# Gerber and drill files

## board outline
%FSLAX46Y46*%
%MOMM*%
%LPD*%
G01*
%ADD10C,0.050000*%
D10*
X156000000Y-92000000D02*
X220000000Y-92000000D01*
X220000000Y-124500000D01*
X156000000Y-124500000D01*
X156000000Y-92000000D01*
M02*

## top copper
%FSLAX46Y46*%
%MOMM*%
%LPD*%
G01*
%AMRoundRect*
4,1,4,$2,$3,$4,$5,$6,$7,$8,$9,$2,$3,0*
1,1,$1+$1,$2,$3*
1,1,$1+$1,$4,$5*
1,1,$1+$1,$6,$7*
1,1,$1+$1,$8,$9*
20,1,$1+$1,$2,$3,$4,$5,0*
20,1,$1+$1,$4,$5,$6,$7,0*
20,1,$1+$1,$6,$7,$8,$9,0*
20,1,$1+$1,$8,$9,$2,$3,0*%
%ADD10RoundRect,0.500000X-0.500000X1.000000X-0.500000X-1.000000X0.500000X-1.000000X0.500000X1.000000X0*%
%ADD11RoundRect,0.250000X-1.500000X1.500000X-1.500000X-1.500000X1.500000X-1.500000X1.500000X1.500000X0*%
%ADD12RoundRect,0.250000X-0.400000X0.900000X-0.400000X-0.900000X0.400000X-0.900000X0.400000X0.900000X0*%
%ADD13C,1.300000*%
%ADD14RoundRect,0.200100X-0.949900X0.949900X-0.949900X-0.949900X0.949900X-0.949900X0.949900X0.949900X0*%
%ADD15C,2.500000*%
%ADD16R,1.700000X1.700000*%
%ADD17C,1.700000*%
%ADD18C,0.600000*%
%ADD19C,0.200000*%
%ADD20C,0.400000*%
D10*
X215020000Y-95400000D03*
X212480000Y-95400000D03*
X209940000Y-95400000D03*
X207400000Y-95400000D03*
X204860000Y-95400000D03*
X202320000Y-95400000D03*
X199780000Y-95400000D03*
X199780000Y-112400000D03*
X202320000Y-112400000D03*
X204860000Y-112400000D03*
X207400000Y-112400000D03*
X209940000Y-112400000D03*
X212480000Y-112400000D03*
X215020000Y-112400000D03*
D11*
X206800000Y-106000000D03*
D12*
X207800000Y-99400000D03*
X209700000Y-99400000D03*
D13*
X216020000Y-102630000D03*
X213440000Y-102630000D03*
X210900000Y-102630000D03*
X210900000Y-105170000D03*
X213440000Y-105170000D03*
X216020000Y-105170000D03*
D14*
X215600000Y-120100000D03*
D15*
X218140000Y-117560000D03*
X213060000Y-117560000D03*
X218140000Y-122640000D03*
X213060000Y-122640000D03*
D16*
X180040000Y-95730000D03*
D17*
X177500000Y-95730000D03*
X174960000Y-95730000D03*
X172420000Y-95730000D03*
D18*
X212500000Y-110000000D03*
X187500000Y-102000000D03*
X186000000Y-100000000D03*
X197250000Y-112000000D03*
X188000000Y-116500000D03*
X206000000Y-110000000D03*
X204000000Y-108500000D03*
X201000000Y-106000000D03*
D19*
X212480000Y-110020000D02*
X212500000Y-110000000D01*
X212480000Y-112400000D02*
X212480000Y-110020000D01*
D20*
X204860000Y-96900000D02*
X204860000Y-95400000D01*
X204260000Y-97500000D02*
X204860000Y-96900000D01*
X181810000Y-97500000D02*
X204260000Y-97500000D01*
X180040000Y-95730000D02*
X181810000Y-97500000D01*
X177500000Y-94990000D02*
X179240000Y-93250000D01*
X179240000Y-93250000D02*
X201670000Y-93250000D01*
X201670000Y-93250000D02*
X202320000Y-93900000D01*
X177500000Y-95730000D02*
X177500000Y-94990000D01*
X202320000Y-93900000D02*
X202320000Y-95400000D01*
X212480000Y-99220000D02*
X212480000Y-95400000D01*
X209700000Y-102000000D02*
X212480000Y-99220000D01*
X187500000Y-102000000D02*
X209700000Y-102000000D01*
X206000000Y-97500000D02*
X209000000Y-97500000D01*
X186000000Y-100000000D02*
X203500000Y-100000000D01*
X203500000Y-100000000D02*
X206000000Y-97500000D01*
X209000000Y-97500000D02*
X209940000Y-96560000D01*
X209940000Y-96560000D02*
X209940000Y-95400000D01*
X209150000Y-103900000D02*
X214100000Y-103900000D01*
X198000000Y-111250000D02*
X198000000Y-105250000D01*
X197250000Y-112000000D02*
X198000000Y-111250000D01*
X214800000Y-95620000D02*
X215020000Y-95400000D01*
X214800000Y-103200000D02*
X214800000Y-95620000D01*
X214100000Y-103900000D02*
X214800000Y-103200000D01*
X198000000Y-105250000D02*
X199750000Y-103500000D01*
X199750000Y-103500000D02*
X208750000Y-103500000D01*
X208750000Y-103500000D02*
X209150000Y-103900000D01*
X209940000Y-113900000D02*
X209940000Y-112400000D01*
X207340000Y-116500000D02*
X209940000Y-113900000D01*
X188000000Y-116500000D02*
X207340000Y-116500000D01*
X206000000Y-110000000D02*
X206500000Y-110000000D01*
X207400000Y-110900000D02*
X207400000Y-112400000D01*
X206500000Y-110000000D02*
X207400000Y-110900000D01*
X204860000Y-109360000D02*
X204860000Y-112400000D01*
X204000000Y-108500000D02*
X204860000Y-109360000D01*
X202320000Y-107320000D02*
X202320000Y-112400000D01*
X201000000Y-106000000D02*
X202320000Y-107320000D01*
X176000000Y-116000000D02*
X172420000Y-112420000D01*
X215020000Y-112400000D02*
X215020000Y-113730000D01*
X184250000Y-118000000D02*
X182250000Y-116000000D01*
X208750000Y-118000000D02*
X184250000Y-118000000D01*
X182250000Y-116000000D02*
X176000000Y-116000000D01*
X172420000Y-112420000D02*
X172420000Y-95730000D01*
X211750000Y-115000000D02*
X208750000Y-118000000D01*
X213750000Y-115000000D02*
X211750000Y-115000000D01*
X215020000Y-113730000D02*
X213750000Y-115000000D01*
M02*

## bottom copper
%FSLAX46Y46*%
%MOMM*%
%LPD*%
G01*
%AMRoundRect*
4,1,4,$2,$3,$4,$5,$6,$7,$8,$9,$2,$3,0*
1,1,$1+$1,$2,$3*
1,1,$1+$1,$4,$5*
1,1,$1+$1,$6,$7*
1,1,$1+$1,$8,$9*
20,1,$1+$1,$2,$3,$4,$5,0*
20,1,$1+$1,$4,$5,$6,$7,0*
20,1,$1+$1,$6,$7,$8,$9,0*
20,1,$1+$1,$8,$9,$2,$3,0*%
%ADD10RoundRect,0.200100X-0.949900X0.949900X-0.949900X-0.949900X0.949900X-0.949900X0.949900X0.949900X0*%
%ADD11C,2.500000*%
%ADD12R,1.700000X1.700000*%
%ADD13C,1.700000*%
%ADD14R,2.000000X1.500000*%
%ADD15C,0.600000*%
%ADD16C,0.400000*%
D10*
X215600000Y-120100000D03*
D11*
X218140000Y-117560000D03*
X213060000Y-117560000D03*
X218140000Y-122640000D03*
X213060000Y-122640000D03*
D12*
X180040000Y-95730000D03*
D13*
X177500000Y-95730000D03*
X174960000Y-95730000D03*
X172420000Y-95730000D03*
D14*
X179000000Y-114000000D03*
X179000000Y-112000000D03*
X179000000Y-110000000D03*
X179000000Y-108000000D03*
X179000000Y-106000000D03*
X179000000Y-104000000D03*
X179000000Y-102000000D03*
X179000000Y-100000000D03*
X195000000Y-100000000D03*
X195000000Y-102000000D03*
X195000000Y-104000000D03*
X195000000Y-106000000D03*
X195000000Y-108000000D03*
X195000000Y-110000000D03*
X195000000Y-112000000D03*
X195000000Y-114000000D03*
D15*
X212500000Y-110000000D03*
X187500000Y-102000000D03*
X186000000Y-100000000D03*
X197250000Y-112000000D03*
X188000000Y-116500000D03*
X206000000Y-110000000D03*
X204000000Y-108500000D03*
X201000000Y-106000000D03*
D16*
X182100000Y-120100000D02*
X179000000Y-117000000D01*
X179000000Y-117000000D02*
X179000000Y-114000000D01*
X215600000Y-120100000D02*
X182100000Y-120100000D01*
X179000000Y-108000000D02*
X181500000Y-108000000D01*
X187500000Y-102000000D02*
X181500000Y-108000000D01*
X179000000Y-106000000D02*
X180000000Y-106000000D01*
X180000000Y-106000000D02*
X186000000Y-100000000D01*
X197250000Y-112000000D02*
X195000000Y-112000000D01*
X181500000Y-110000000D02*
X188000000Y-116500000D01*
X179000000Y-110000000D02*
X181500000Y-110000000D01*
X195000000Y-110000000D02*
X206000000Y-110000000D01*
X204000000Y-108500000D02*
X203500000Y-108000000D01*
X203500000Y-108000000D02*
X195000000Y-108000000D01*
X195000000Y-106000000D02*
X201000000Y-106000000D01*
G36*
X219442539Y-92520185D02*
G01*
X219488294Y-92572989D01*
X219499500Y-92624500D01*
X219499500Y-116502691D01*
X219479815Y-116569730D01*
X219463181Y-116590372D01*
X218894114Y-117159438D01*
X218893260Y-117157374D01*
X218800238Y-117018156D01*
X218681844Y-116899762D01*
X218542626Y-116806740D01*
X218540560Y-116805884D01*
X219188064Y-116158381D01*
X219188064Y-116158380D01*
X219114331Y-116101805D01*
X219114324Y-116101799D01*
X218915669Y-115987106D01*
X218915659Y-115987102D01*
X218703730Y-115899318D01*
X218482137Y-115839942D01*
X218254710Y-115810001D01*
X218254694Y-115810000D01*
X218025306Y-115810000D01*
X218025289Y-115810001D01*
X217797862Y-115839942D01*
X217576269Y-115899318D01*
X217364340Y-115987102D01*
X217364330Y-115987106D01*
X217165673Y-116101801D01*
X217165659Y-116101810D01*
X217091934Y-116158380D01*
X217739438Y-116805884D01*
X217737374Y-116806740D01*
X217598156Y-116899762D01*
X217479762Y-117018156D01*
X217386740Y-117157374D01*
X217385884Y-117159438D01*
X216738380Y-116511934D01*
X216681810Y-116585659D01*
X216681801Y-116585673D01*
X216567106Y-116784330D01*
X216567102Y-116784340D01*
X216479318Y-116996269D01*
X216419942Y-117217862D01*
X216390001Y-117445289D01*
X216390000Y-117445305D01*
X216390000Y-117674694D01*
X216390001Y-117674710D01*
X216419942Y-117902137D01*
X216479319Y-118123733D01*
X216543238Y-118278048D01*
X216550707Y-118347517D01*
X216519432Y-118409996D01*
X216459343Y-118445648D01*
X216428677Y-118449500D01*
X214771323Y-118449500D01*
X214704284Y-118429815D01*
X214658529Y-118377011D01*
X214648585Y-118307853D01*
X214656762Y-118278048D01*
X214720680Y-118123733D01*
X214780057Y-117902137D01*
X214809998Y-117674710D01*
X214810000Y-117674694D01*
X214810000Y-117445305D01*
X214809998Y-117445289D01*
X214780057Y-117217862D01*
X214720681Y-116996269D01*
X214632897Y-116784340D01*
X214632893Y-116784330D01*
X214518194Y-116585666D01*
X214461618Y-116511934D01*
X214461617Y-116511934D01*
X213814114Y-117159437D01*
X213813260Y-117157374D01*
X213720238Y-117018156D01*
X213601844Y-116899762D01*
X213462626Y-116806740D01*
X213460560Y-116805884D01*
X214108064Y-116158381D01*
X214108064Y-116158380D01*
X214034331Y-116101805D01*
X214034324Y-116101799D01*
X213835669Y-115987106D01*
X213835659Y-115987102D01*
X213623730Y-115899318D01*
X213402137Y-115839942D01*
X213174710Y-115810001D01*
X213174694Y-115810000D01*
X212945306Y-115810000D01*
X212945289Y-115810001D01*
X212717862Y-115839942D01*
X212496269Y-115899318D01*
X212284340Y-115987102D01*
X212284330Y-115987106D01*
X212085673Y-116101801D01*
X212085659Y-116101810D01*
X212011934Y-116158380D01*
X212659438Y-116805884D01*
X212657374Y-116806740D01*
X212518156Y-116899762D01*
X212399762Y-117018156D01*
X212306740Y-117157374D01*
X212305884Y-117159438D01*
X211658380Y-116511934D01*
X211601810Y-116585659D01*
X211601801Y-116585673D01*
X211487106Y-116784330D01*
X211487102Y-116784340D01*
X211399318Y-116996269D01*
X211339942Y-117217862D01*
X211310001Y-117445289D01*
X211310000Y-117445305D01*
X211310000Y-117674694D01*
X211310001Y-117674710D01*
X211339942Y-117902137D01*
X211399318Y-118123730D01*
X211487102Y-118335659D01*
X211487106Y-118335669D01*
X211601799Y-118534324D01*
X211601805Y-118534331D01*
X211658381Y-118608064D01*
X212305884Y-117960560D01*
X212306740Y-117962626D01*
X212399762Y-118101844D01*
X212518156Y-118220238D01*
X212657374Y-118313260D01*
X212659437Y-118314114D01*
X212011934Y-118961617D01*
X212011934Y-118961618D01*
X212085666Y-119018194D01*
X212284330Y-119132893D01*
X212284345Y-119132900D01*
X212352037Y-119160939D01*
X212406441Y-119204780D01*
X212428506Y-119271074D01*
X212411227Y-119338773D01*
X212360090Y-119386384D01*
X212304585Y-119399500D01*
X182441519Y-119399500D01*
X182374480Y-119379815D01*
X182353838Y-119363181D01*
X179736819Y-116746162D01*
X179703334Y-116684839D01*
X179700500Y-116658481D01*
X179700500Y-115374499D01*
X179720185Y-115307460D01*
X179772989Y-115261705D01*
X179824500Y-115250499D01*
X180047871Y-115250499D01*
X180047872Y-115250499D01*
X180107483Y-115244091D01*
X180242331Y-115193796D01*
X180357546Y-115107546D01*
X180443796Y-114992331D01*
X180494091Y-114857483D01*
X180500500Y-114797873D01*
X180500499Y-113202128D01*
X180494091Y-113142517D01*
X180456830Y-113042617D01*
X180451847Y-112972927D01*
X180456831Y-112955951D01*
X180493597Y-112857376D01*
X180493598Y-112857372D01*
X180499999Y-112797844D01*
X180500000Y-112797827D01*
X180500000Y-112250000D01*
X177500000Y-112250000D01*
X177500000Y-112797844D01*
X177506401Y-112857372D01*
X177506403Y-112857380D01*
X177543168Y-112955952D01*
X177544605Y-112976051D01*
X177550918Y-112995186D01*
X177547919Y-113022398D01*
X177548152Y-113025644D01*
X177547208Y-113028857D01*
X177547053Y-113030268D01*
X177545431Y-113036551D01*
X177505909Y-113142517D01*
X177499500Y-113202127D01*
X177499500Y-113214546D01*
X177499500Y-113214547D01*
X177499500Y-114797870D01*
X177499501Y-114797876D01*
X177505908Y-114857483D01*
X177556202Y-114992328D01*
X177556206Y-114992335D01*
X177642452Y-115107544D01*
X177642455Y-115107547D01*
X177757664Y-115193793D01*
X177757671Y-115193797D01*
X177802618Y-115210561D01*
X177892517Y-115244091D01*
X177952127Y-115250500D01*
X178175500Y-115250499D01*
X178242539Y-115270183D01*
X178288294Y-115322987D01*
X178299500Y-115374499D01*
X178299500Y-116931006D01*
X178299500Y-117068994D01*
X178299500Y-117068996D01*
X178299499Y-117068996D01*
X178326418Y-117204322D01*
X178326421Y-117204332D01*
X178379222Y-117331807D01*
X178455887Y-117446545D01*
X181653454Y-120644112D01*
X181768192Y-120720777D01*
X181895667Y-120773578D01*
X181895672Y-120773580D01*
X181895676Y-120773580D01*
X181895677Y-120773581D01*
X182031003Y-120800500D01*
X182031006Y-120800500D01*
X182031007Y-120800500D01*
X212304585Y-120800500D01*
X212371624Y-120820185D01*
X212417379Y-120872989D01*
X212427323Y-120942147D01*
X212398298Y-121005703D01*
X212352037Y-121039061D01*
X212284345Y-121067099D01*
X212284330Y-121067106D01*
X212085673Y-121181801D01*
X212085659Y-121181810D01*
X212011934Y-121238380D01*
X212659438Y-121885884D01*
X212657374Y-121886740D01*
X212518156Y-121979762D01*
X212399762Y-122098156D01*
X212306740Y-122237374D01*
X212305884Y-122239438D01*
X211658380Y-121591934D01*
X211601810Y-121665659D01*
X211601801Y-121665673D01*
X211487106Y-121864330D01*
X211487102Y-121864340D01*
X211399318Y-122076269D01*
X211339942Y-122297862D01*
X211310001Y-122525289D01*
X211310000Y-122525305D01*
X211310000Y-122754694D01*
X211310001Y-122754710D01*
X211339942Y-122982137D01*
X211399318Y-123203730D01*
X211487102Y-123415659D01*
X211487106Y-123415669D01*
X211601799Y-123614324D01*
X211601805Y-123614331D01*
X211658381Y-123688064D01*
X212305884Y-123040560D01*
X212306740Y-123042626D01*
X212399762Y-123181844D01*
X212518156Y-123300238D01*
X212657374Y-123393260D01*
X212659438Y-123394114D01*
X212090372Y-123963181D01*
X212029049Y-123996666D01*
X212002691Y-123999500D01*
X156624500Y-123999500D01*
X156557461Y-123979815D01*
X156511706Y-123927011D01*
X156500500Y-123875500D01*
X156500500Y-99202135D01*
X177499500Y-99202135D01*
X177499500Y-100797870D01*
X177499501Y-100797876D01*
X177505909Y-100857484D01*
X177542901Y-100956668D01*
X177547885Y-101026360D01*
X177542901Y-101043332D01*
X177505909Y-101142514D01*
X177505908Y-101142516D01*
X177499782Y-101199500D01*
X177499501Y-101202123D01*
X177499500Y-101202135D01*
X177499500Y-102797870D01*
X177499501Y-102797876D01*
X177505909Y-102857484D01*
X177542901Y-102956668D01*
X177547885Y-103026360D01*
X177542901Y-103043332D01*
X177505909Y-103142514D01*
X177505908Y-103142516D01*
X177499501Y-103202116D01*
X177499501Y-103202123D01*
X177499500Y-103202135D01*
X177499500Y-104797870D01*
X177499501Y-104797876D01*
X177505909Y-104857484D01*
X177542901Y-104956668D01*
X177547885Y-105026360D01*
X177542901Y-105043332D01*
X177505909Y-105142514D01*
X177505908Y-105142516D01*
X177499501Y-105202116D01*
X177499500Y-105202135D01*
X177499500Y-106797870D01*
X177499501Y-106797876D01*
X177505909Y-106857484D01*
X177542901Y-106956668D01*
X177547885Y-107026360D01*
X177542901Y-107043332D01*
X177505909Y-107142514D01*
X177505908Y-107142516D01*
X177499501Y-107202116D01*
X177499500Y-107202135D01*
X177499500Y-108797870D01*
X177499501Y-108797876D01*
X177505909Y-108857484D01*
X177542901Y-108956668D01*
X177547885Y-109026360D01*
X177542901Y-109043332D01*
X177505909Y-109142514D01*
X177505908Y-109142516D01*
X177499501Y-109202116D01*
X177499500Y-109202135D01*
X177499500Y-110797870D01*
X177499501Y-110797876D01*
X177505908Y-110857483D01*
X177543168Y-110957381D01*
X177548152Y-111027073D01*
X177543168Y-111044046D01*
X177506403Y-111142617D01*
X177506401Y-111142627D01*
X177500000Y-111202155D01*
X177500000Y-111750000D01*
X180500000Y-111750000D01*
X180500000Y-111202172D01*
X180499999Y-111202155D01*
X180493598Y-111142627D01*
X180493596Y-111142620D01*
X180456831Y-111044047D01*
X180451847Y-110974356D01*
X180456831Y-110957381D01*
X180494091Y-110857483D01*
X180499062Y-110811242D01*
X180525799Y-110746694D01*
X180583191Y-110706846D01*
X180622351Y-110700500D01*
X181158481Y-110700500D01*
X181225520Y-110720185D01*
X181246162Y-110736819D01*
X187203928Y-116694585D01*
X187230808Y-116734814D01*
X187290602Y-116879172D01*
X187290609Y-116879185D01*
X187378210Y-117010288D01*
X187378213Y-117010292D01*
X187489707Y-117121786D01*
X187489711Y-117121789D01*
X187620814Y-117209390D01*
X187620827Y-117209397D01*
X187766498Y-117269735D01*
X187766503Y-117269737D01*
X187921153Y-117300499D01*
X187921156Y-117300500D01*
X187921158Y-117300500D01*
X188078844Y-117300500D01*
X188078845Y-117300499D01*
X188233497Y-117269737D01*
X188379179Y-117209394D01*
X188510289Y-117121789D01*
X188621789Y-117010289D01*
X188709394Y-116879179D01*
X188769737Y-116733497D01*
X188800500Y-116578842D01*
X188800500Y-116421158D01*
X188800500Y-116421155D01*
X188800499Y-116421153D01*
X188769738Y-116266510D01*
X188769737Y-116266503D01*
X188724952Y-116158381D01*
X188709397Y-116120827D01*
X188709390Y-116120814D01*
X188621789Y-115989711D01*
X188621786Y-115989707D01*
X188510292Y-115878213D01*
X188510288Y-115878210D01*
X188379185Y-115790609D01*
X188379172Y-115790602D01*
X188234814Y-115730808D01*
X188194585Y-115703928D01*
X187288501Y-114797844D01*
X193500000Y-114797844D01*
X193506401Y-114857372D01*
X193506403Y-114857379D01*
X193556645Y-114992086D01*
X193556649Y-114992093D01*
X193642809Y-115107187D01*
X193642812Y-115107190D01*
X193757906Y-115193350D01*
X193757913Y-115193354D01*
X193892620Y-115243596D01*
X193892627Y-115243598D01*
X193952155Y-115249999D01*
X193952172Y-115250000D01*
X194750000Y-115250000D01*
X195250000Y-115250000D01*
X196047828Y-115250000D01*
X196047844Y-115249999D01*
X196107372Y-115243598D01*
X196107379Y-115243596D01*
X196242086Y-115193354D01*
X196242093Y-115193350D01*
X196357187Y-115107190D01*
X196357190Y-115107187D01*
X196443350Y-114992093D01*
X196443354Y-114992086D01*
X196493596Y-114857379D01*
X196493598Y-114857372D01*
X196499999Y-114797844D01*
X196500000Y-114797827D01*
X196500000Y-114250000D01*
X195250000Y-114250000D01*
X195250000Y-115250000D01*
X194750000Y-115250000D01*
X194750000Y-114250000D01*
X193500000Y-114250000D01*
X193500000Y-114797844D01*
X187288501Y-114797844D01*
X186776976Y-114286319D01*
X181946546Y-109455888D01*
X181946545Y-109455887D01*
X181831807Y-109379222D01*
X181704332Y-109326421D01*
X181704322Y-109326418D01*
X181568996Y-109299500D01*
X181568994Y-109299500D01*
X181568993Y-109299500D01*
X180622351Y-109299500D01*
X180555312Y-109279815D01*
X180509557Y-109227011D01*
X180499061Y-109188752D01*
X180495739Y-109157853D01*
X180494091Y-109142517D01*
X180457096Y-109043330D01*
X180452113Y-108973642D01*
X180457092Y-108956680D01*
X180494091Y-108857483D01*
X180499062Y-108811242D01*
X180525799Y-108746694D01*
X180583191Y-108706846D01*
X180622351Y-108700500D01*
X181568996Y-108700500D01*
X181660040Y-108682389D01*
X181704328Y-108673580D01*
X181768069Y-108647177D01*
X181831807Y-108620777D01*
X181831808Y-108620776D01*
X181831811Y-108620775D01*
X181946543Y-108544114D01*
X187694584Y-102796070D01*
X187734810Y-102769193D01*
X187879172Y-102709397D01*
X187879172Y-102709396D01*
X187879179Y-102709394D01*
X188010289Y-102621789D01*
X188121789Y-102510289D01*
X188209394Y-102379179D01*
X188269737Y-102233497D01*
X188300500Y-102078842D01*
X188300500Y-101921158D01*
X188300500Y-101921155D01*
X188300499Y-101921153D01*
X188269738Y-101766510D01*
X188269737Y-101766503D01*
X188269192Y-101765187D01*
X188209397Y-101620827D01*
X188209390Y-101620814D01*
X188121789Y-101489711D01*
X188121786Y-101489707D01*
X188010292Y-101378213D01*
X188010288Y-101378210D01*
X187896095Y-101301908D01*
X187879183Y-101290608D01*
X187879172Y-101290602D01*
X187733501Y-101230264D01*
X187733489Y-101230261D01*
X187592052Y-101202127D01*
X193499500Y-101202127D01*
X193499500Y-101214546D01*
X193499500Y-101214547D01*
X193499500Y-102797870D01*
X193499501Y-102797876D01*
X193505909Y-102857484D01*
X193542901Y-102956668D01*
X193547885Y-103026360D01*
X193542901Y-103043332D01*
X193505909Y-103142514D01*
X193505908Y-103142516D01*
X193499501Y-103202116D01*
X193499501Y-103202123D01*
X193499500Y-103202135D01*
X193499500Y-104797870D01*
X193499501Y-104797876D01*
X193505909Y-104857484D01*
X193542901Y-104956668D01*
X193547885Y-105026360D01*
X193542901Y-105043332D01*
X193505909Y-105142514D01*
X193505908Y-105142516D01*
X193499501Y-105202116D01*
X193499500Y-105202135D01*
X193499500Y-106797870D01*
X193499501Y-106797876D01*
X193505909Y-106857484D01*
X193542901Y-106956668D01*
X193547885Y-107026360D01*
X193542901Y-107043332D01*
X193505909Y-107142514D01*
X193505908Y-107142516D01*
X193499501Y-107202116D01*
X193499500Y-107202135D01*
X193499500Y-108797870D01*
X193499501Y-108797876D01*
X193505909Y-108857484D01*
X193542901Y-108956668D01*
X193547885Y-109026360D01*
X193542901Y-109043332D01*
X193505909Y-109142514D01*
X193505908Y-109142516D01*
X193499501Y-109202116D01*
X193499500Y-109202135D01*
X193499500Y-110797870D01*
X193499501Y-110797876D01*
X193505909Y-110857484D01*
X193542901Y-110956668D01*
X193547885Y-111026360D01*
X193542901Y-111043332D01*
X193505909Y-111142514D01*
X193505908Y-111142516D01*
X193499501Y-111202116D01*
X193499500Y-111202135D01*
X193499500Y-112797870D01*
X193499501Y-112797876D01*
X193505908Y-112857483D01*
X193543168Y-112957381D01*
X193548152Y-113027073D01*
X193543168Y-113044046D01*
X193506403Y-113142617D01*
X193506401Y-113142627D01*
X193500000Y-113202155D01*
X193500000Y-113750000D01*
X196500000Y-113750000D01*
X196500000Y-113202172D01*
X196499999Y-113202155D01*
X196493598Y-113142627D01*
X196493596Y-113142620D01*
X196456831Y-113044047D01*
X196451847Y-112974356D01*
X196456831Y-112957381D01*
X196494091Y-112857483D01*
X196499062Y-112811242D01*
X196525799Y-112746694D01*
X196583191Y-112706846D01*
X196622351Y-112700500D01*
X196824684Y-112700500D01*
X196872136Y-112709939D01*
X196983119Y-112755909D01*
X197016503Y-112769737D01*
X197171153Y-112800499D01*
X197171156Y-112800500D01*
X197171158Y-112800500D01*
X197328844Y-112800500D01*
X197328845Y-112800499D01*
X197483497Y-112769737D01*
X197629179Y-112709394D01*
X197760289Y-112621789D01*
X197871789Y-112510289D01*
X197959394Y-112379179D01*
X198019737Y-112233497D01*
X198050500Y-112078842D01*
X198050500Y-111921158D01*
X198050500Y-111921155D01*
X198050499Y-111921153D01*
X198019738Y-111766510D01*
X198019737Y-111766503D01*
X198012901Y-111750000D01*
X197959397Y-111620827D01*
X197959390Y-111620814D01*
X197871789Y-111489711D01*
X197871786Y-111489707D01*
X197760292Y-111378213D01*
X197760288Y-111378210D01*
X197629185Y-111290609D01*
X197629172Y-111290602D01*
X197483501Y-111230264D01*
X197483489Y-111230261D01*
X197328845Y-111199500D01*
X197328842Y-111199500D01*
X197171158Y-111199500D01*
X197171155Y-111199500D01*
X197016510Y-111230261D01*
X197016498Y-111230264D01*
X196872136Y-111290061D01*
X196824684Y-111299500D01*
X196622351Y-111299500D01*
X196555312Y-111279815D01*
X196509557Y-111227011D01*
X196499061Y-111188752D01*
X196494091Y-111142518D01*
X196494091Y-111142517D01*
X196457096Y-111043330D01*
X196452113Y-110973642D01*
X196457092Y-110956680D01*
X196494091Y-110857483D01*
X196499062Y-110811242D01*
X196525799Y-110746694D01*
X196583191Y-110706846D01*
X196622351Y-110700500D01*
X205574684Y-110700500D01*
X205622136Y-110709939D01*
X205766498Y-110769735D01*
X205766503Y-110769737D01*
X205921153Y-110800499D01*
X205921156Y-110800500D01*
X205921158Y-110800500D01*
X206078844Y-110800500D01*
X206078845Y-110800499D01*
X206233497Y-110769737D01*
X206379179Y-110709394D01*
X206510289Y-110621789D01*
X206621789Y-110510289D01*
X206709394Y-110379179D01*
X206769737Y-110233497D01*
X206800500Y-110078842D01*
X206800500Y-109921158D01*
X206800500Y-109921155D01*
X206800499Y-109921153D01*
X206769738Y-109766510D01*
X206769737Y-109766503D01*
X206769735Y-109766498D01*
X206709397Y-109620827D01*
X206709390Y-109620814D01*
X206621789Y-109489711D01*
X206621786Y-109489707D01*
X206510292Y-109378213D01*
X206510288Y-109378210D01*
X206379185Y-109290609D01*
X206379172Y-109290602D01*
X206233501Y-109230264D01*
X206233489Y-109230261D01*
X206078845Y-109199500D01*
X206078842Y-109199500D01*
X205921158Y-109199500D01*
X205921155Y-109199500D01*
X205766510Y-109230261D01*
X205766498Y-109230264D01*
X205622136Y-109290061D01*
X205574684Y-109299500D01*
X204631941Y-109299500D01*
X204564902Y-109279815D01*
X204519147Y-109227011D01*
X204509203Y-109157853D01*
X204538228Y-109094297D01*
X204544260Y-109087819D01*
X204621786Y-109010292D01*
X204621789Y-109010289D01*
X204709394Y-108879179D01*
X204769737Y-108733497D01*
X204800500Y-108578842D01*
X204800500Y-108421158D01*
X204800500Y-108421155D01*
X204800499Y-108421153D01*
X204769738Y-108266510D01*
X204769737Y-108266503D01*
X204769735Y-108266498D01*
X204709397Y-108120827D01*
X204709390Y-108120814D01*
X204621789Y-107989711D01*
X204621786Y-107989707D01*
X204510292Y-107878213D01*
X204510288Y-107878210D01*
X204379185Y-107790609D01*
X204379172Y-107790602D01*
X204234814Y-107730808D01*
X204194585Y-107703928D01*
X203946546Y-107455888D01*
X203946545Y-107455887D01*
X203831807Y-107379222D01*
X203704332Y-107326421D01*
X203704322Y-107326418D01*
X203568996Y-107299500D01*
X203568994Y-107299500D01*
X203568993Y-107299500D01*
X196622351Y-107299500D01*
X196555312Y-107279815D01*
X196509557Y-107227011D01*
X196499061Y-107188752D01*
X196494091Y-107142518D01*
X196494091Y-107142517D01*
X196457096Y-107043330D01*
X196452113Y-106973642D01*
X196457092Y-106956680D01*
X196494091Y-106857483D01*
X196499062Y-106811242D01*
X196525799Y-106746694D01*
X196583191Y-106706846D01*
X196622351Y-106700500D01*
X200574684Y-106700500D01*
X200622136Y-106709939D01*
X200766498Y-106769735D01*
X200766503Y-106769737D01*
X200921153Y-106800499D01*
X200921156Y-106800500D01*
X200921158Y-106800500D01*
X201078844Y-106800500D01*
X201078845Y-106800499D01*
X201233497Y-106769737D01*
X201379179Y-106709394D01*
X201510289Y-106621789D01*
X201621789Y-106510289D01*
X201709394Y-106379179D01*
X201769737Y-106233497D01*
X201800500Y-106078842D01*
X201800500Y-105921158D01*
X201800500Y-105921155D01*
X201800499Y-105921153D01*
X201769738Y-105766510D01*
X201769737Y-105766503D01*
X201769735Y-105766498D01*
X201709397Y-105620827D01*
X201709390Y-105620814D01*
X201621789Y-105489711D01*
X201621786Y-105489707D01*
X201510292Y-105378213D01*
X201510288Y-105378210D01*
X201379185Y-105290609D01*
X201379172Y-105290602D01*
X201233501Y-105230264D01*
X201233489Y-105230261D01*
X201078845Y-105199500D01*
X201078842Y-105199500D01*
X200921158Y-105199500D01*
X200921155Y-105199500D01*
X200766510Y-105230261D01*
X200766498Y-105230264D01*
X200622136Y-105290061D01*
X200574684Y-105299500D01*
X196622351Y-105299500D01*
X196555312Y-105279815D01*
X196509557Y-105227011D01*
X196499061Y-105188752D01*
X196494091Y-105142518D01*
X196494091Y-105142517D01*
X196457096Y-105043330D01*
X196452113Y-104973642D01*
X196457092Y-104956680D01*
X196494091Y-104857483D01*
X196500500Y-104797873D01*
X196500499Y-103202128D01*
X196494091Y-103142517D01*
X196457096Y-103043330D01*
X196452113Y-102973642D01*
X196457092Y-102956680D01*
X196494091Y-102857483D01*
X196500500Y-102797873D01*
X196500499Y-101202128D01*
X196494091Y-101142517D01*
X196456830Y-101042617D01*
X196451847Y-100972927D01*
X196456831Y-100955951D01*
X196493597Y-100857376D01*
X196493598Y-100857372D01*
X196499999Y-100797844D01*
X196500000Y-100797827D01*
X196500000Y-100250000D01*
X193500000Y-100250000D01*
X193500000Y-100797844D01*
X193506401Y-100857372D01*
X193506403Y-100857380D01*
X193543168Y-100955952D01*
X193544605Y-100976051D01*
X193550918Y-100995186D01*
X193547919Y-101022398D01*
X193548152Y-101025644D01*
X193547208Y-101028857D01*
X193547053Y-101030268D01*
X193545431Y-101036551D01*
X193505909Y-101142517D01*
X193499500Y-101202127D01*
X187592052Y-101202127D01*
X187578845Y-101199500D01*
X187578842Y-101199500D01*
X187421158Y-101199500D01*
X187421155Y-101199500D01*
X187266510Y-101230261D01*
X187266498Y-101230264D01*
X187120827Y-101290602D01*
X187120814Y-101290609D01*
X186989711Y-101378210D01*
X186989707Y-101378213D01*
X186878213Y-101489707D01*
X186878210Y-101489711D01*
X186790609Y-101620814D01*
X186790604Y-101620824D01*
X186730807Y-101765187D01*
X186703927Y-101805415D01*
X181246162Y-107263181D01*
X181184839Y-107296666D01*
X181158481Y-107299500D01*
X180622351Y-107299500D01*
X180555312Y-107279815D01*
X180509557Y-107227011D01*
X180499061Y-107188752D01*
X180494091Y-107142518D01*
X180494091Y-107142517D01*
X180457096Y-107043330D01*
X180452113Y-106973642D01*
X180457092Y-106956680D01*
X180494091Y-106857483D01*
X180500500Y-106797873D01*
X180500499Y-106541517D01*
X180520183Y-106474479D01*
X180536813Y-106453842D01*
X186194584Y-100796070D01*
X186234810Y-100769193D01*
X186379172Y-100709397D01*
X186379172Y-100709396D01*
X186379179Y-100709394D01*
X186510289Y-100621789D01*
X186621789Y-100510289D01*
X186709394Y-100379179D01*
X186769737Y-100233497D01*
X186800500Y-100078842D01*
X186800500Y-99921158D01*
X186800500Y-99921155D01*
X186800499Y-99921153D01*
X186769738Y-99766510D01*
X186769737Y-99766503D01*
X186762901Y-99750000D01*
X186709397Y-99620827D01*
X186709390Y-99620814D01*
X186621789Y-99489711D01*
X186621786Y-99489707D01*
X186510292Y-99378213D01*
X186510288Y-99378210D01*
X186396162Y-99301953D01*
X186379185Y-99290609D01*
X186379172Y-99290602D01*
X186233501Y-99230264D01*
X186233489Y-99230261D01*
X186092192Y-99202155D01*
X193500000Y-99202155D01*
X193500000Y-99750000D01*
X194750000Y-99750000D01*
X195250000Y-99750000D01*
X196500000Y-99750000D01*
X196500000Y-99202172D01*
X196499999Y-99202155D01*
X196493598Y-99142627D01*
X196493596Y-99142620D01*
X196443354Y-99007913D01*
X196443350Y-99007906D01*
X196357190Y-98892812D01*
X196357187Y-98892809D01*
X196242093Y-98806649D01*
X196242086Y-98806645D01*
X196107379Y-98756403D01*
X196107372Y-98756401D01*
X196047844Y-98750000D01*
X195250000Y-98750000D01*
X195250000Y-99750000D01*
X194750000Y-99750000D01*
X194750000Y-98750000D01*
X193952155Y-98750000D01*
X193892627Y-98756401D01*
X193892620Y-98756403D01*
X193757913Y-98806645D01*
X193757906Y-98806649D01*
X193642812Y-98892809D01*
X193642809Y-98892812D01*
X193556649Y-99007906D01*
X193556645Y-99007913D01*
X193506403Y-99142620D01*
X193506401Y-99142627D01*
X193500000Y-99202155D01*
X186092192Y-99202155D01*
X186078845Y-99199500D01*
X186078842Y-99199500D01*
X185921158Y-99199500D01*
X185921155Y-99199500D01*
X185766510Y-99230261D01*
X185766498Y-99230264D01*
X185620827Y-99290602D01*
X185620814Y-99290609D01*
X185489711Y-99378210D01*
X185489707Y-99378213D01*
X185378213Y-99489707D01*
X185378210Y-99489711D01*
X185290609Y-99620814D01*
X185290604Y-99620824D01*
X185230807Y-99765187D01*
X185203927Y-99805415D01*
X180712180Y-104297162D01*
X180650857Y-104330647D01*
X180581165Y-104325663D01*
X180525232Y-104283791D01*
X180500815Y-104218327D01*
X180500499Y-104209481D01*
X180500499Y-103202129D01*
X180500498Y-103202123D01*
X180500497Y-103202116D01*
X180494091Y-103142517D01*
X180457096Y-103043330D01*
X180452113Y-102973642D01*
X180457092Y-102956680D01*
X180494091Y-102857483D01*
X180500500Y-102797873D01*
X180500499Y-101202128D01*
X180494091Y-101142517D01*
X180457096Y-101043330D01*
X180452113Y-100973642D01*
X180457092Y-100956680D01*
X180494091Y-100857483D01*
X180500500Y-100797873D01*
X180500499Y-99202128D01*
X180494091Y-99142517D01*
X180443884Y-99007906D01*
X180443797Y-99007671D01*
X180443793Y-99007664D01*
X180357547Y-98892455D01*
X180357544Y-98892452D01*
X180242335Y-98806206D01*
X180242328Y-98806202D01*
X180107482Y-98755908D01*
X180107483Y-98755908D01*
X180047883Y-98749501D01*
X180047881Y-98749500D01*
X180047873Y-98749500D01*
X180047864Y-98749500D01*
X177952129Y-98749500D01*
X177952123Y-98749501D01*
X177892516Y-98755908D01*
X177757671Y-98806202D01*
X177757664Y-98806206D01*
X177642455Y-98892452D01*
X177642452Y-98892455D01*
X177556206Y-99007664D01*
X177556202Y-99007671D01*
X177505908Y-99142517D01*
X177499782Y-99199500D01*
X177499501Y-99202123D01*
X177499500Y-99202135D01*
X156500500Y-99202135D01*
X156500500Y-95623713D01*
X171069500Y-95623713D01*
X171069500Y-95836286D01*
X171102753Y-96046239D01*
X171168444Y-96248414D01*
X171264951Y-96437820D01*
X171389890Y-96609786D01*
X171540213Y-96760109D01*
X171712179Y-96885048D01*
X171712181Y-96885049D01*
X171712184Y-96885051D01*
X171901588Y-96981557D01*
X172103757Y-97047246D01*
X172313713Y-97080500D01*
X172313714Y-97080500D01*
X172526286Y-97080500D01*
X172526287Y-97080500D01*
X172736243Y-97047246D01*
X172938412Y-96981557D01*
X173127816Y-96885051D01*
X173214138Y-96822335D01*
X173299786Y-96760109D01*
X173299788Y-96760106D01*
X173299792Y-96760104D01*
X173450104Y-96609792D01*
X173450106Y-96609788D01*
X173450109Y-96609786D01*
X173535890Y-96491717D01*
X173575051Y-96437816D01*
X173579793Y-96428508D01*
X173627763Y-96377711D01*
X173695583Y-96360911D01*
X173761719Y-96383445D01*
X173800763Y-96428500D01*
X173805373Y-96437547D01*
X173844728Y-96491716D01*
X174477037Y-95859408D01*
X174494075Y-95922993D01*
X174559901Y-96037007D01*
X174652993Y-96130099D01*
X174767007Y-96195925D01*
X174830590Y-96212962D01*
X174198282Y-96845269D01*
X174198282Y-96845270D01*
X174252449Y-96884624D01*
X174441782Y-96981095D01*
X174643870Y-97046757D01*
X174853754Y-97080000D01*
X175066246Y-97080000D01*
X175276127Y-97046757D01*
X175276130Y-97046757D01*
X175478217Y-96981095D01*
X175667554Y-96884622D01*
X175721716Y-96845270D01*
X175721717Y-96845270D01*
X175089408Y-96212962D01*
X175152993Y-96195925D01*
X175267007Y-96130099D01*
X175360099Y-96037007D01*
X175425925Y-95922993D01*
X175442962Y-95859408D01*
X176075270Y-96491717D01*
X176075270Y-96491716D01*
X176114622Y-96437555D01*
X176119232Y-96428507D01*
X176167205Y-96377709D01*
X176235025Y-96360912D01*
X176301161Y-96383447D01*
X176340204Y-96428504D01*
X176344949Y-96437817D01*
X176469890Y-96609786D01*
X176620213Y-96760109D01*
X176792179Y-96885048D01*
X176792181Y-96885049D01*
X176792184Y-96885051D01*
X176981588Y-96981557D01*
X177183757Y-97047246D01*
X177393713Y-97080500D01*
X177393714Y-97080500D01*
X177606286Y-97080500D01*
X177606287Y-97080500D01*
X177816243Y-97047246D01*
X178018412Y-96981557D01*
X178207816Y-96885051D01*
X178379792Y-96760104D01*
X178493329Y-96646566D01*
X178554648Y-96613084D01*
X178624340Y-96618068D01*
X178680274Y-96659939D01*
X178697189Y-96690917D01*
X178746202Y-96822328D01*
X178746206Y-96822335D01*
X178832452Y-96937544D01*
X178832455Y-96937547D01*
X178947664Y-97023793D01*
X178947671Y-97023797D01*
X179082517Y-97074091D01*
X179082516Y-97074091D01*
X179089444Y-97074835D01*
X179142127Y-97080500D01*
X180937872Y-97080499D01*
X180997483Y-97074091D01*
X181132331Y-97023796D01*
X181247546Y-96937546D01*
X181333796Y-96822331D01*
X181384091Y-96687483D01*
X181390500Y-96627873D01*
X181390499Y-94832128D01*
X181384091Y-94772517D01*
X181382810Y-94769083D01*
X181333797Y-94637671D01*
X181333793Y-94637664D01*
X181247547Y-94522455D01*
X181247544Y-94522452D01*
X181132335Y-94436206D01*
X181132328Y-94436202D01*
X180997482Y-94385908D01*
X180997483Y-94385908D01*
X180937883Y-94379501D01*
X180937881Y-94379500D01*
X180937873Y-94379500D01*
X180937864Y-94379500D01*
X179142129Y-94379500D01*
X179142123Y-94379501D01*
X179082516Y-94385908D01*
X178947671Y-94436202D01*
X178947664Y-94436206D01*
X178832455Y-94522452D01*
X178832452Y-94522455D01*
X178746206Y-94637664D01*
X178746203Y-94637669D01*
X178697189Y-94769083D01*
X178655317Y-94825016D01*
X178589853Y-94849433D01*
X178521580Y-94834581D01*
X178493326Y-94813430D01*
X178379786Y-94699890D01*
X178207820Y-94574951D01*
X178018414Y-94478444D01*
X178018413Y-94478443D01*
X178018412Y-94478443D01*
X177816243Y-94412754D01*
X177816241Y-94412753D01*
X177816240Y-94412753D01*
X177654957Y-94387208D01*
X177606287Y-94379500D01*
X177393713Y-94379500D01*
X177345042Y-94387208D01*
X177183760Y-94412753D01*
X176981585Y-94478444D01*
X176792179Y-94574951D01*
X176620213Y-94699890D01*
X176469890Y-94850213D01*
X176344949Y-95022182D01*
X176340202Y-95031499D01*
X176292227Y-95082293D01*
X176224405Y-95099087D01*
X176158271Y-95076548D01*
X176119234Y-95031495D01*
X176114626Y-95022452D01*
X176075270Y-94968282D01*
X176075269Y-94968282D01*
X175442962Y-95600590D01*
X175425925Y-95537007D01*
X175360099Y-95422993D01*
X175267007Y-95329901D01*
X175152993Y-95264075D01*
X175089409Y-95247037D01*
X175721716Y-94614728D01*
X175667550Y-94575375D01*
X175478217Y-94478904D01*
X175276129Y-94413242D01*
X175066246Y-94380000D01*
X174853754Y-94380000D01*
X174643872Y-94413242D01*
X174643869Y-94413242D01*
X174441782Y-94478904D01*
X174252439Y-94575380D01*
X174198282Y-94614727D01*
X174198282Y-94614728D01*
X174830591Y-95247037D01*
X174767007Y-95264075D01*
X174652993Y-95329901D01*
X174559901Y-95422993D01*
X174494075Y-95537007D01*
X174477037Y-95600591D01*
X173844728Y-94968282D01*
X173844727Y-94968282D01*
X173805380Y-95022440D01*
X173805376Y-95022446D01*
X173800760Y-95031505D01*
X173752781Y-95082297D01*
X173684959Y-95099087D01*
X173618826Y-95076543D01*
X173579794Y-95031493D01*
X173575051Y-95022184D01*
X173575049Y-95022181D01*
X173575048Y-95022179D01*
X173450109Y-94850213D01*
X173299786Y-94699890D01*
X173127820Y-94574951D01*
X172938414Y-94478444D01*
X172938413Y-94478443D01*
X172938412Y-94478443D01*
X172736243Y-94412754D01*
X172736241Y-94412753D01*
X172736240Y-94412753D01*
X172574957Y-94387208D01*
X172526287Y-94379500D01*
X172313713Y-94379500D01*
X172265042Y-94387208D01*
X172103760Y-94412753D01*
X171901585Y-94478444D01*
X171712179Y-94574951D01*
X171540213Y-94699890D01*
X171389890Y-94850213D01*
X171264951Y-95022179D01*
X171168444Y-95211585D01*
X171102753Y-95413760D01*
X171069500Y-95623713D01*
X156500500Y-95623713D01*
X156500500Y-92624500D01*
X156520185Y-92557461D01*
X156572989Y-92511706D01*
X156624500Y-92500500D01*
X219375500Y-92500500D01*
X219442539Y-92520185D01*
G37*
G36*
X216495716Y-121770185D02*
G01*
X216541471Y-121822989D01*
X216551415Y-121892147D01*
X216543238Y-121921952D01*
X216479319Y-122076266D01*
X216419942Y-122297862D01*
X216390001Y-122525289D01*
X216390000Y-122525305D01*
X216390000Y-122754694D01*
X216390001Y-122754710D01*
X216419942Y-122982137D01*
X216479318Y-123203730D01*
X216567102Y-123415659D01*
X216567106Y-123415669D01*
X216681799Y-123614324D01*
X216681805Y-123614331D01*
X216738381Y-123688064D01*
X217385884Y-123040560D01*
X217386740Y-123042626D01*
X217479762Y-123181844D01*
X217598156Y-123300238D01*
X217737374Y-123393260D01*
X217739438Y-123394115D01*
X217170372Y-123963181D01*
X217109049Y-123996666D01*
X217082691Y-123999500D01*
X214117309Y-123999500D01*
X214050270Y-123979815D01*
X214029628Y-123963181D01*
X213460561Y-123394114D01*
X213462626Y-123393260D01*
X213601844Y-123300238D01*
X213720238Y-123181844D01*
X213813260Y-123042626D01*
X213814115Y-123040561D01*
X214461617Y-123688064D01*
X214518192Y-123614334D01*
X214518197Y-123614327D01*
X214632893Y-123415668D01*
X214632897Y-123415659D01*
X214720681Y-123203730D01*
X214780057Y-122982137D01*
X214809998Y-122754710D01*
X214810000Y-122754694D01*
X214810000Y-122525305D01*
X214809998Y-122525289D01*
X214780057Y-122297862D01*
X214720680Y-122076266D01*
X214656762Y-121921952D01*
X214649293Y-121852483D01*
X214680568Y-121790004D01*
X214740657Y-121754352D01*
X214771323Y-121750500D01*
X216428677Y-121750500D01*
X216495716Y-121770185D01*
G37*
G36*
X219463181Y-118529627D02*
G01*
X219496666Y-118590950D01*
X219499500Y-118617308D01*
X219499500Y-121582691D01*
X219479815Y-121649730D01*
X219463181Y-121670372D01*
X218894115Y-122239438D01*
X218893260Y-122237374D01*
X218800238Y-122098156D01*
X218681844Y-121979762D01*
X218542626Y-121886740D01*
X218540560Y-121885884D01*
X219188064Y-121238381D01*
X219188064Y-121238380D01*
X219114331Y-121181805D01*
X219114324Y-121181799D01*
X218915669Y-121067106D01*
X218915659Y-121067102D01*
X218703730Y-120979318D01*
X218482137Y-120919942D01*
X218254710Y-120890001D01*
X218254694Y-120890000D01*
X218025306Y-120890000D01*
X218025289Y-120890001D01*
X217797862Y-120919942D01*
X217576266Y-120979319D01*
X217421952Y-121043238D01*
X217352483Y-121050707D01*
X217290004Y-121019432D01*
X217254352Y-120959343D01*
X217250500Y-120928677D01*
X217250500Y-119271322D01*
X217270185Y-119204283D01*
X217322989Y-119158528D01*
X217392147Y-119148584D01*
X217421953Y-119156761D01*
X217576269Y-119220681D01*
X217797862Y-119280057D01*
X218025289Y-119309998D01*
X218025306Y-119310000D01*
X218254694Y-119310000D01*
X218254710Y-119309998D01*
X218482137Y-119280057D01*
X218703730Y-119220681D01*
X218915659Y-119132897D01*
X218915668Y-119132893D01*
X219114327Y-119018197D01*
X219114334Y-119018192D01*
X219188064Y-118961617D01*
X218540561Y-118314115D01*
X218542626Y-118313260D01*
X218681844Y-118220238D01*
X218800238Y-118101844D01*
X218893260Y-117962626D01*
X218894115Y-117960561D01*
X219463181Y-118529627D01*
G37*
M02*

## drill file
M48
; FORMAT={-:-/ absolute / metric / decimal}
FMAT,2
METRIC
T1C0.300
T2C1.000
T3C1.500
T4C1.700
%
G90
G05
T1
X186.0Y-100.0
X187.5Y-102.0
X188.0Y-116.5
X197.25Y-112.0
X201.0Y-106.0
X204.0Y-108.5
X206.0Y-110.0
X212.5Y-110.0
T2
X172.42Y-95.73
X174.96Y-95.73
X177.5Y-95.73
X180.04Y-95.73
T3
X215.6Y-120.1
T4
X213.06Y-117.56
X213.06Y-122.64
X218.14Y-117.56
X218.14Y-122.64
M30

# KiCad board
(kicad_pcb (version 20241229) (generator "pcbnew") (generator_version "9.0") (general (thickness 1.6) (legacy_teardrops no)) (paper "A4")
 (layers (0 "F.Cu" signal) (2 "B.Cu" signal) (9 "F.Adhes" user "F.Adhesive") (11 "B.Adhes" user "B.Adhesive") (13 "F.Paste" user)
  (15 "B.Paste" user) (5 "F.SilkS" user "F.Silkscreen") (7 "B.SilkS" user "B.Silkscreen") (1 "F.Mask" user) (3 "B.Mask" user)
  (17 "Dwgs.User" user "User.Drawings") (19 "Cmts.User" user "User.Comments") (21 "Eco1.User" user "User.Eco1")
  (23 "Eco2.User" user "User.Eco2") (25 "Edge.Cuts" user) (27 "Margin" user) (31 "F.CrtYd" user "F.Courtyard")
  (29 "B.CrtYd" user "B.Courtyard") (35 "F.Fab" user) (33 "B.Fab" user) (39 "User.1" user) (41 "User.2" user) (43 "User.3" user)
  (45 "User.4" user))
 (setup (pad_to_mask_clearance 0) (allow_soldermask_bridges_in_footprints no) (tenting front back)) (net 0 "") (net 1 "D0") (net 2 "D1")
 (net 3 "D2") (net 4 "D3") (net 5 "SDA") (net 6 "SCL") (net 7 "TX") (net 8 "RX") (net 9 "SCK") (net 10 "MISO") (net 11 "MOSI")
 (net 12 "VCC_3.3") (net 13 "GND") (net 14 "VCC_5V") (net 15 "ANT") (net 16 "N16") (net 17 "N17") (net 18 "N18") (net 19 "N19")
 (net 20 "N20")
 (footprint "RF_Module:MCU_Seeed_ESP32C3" (layer "F.Cu") (at 207.4 103.9 -90)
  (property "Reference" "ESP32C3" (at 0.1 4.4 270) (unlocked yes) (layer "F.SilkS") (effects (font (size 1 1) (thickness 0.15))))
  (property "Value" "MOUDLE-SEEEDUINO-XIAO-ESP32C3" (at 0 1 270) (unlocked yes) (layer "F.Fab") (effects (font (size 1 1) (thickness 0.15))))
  (pad "" smd roundrect (at 1.1 -0.4 270) (size 1.5 1.5) (layers "F.Paste") (roundrect_rratio 0.1666666667))
  (pad "" smd roundrect (at 1.1 1.6 270) (size 1.5 1.5) (layers "F.Paste") (roundrect_rratio 0.1666666667))
  (pad "" smd roundrect (at 3.1 -0.4 270) (size 1.5 1.5) (layers "F.Paste") (roundrect_rratio 0.1666666667))
  (pad "" smd roundrect (at 3.1 1.6 270) (size 1.5 1.5) (layers "F.Paste") (roundrect_rratio 0.1666666667))
  (pad "1" smd roundrect (at -8.5 -7.62 270) (size 3 2) (layers "F.Cu" "F.Mask" "F.Paste") (roundrect_rratio 0.25) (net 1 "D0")
   (thermal_bridge_angle 45))
  (pad "2" smd roundrect (at -8.5 -5.08 270) (size 3 2) (layers "F.Cu" "F.Mask" "F.Paste") (roundrect_rratio 0.25) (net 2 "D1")
   (thermal_bridge_angle 45))
  (pad "3" smd roundrect (at -8.5 -2.54 270) (size 3 2) (layers "F.Cu" "F.Mask" "F.Paste") (roundrect_rratio 0.25) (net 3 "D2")
   (thermal_bridge_angle 45))
  (pad "4" smd roundrect (at -8.5 0 270) (size 3 2) (layers "F.Cu" "F.Mask" "F.Paste") (roundrect_rratio 0.25) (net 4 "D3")
   (thermal_bridge_angle 45))
  (pad "5" smd roundrect (at -8.5 2.54 270) (size 3 2) (layers "F.Cu" "F.Mask" "F.Paste") (roundrect_rratio 0.25) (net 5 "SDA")
   (thermal_bridge_angle 45))
  (pad "6" smd roundrect (at -8.5 5.08 270) (size 3 2) (layers "F.Cu" "F.Mask" "F.Paste") (roundrect_rratio 0.25) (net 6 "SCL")
   (thermal_bridge_angle 45))
  (pad "7" smd roundrect (at -8.5 7.62 270) (size 3 2) (layers "F.Cu" "F.Mask" "F.Paste") (roundrect_rratio 0.25) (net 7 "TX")
   (thermal_bridge_angle 45))
  (pad "8" smd roundrect (at 8.5 7.62 270) (size 3 2) (layers "F.Cu" "F.Mask" "F.Paste") (roundrect_rratio 0.25) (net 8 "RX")
   (thermal_bridge_angle 45))
  (pad "9" smd roundrect (at 8.5 5.08 270) (size 3 2) (layers "F.Cu" "F.Mask" "F.Paste") (roundrect_rratio 0.25) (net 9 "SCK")
   (thermal_bridge_angle 45))
  (pad "10" smd roundrect (at 8.5 2.54 270) (size 3 2) (layers "F.Cu" "F.Mask" "F.Paste") (roundrect_rratio 0.25) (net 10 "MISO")
   (thermal_bridge_angle 45))
  (pad "11" smd roundrect (at 8.5 0 270) (size 3 2) (layers "F.Cu" "F.Mask" "F.Paste") (roundrect_rratio 0.25) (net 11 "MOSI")
   (thermal_bridge_angle 45))
  (pad "12" smd roundrect (at 8.5 -2.54 270) (size 3 2) (layers "F.Cu" "F.Mask" "F.Paste") (roundrect_rratio 0.25) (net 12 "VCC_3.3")
   (thermal_bridge_angle 45))
  (pad "13" smd roundrect (at 8.5 -5.08 270) (size 3 2) (layers "F.Cu" "F.Mask" "F.Paste") (roundrect_rratio 0.25) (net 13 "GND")
   (thermal_bridge_angle 45))
  (pad "14" smd roundrect (at 8.5 -7.62 270) (size 3 2) (layers "F.Cu" "F.Mask" "F.Paste") (roundrect_rratio 0.25) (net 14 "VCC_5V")
   (thermal_bridge_angle 45))
  (pad "15" smd roundrect (at 2.1 0.6 270) (size 3.5 3.5) (layers "F.Cu" "F.Mask") (roundrect_rratio 0.07142857143))
  (pad "16" smd roundrect (at -4.5 -0.4 270) (size 2.3 1.3) (layers "F.Cu" "F.Mask" "F.Paste") (roundrect_rratio 0.1923076923))
  (pad "17" smd roundrect (at -4.5 -2.3 270) (size 2.3 1.3) (layers "F.Cu" "F.Mask" "F.Paste") (roundrect_rratio 0.1923076923))
  (pad "18" smd circle (at -1.27 -8.62 270) (size 1.3 1.3) (layers "F.Cu" "F.Mask" "F.Paste"))
  (pad "19" smd circle (at -1.27 -6.04 270) (size 1.3 1.3) (layers "F.Cu" "F.Mask" "F.Paste"))
  (pad "20" smd circle (at -1.27 -3.5 270) (size 1.3 1.3) (layers "F.Cu" "F.Mask" "F.Paste"))
  (pad "21" smd circle (at 1.27 -3.5 270) (size 1.3 1.3) (layers "F.Cu" "F.Mask" "F.Paste"))
  (pad "22" smd circle (at 1.27 -6.04 270) (size 1.3 1.3) (layers "F.Cu" "F.Mask" "F.Paste"))
  (pad "23" smd circle (at 1.27 -8.62 270) (size 1.3 1.3) (layers "F.Cu" "F.Mask" "F.Paste")))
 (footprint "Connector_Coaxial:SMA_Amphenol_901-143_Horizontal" (layer "F.Cu") (at 215.6 120.1 -90)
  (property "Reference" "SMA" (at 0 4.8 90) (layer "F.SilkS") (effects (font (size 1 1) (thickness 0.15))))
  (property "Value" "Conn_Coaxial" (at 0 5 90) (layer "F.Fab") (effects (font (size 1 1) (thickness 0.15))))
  (pad "1" thru_hole roundrect (at 0 0 270) (size 2.3 2.3) (drill 1.5) (layers "*.Cu" "*.Mask") (remove_unused_layers yes)
   (keep_end_layers yes) (zone_layer_connections) (roundrect_rratio 0.087) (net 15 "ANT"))
  (pad "2" thru_hole circle (at -2.54 -2.54 270) (size 2.5 2.5) (drill 1.7) (layers "*.Cu" "*.Mask") (remove_unused_layers yes)
   (keep_end_layers yes) (zone_layer_connections) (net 13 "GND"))
  (pad "2" thru_hole circle (at -2.54 2.54 270) (size 2.5 2.5) (drill 1.7) (layers "*.Cu" "*.Mask") (remove_unused_layers yes)
   (keep_end_layers yes) (zone_layer_connections) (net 13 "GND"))
  (pad "2" thru_hole circle (at 2.54 -2.54 270) (size 2.5 2.5) (drill 1.7) (layers "*.Cu" "*.Mask") (remove_unused_layers yes)
   (keep_end_layers yes) (zone_layer_connections) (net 13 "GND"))
  (pad "2" thru_hole circle (at 2.54 2.54 270) (size 2.5 2.5) (drill 1.7) (layers "*.Cu" "*.Mask") (remove_unused_layers yes)
   (keep_end_layers yes) (zone_layer_connections) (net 13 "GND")))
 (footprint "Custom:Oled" (layer "F.Cu") (at 176 102)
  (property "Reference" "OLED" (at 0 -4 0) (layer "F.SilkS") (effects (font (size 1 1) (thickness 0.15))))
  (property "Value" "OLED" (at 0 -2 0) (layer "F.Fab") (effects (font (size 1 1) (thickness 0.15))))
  (pad "1" thru_hole rect (at 4.04 -6.27 270) (size 1.7 1.7) (drill 1) (layers "*.Cu" "*.Mask") (remove_unused_layers no) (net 5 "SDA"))
  (pad "2" thru_hole circle (at 1.5 -6.27 270) (size 1.7 1.7) (drill 1) (layers "*.Cu" "*.Mask") (remove_unused_layers no) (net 6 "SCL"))
  (pad "3" thru_hole circle (at -1.04 -6.27 270) (size 1.7 1.7) (drill 1) (layers "*.Cu" "*.Mask") (remove_unused_layers no) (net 13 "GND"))
  (pad "4" thru_hole circle (at -3.58 -6.27 270) (size 1.7 1.7) (drill 1) (layers "*.Cu" "*.Mask") (remove_unused_layers no)
   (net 14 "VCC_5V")))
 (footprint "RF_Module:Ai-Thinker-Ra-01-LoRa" (layer "B.Cu") (at 187 107)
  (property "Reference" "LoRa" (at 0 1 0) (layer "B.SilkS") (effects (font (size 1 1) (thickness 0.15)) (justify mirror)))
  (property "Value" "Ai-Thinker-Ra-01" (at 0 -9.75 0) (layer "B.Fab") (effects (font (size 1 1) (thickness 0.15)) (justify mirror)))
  (pad "1" smd rect (at -8 7) (size 2 1.5) (layers "B.Cu" "B.Mask" "B.Paste") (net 15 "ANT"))
  (pad "2" smd rect (at -8 5) (size 2 1.5) (layers "B.Cu" "B.Mask" "B.Paste") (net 13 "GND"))
  (pad "3" smd rect (at -8 3) (size 2 1.5) (layers "B.Cu" "B.Mask" "B.Paste") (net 12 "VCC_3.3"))
  (pad "4" smd rect (at -8 1) (size 2 1.5) (layers "B.Cu" "B.Mask" "B.Paste") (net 2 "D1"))
  (pad "5" smd rect (at -8 -1) (size 2 1.5) (layers "B.Cu" "B.Mask" "B.Paste") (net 3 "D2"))
  (pad "6" smd rect (at -8 -3) (size 2 1.5) (layers "B.Cu" "B.Mask" "B.Paste") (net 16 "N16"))
  (pad "7" smd rect (at -8 -5) (size 2 1.5) (layers "B.Cu" "B.Mask" "B.Paste") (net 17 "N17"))
  (pad "8" smd rect (at -8 -7) (size 2 1.5) (layers "B.Cu" "B.Mask" "B.Paste") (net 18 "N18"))
  (pad "9" smd rect (at 8 -7) (size 2 1.5) (layers "B.Cu" "B.Mask" "B.Paste") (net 13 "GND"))
  (pad "10" smd rect (at 8 -5) (size 2 1.5) (layers "B.Cu" "B.Mask" "B.Paste") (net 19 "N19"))
  (pad "11" smd rect (at 8 -3) (size 2 1.5) (layers "B.Cu" "B.Mask" "B.Paste") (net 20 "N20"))
  (pad "12" smd rect (at 8 -1) (size 2 1.5) (layers "B.Cu" "B.Mask" "B.Paste") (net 9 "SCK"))
  (pad "13" smd rect (at 8 1) (size 2 1.5) (layers "B.Cu" "B.Mask" "B.Paste") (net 10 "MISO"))
  (pad "14" smd rect (at 8 3) (size 2 1.5) (layers "B.Cu" "B.Mask" "B.Paste") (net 11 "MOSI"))
  (pad "15" smd rect (at 8 5) (size 2 1.5) (layers "B.Cu" "B.Mask" "B.Paste") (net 1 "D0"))
  (pad "16" smd rect (at 8 7) (size 2 1.5) (layers "B.Cu" "B.Mask" "B.Paste") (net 13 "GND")))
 (gr_rect (start 156 92) (end 220 124.5) (stroke (width 0.05) (type default)) (fill no) (layer "Edge.Cuts"))
 (segment (start 212.48 110.02) (end 212.5 110) (width 0.2) (layer "F.Cu") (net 13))
 (segment (start 212.48 112.4) (end 212.48 110.02) (width 0.2) (layer "F.Cu") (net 13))
 (via (at 212.5 110) (size 0.6) (drill 0.3) (layers "F.Cu" "B.Cu") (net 13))
 (segment (start 182.1 120.1) (end 179 117) (width 0.4) (layer "B.Cu") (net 15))
 (segment (start 179 117) (end 179 114) (width 0.4) (layer "B.Cu") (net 15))
 (segment (start 215.6 120.1) (end 182.1 120.1) (width 0.4) (layer "B.Cu") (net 15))
 (segment (start 204.86 96.9) (end 204.86 95.4) (width 0.4) (layer "F.Cu") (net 5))
 (segment (start 204.26 97.5) (end 204.86 96.9) (width 0.4) (layer "F.Cu") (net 5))
 (segment (start 181.81 97.5) (end 204.26 97.5) (width 0.4) (layer "F.Cu") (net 5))
 (segment (start 180.04 95.73) (end 181.81 97.5) (width 0.4) (layer "F.Cu") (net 5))
 (segment (start 177.5 94.99) (end 179.24 93.25) (width 0.4) (layer "F.Cu") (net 6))
 (segment (start 179.24 93.25) (end 201.67 93.25) (width 0.4) (layer "F.Cu") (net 6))
 (segment (start 201.67 93.25) (end 202.32 93.9) (width 0.4) (layer "F.Cu") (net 6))
 (segment (start 177.5 95.73) (end 177.5 94.99) (width 0.4) (layer "F.Cu") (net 6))
 (segment (start 202.32 93.9) (end 202.32 95.4) (width 0.4) (layer "F.Cu") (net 6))
 (segment (start 212.48 99.22) (end 212.48 95.4) (width 0.4) (layer "F.Cu") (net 2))
 (segment (start 209.7 102) (end 212.48 99.22) (width 0.4) (layer "F.Cu") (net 2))
 (segment (start 187.5 102) (end 209.7 102) (width 0.4) (layer "F.Cu") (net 2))
 (via (at 187.5 102) (size 0.6) (drill 0.3) (layers "F.Cu" "B.Cu") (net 2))
 (segment (start 179 108) (end 181.5 108) (width 0.4) (layer "B.Cu") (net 2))
 (segment (start 187.5 102) (end 181.5 108) (width 0.4) (layer "B.Cu") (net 2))
 (segment (start 206 97.5) (end 209 97.5) (width 0.4) (layer "F.Cu") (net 3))
 (segment (start 186 100) (end 203.5 100) (width 0.4) (layer "F.Cu") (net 3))
 (segment (start 203.5 100) (end 206 97.5) (width 0.4) (layer "F.Cu") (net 3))
 (segment (start 209 97.5) (end 209.94 96.56) (width 0.4) (layer "F.Cu") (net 3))
 (segment (start 209.94 96.56) (end 209.94 95.4) (width 0.4) (layer "F.Cu") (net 3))
 (via (at 186 100) (size 0.6) (drill 0.3) (layers "F.Cu" "B.Cu") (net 3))
 (segment (start 179 106) (end 180 106) (width 0.4) (layer "B.Cu") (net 3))
 (segment (start 180 106) (end 186 100) (width 0.4) (layer "B.Cu") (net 3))
 (segment (start 209.15 103.9) (end 214.1 103.9) (width 0.4) (layer "F.Cu") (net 1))
 (segment (start 198 111.25) (end 198 105.25) (width 0.4) (layer "F.Cu") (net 1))
 (segment (start 197.25 112) (end 198 111.25) (width 0.4) (layer "F.Cu") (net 1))
 (segment (start 214.8 95.62) (end 215.02 95.4) (width 0.4) (layer "F.Cu") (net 1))
 (segment (start 214.8 103.2) (end 214.8 95.62) (width 0.4) (layer "F.Cu") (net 1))
 (segment (start 214.1 103.9) (end 214.8 103.2) (width 0.4) (layer "F.Cu") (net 1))
 (segment (start 198 105.25) (end 199.75 103.5) (width 0.4) (layer "F.Cu") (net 1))
 (segment (start 199.75 103.5) (end 208.75 103.5) (width 0.4) (layer "F.Cu") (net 1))
 (segment (start 208.75 103.5) (end 209.15 103.9) (width 0.4) (layer "F.Cu") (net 1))
 (via (at 197.25 112) (size 0.6) (drill 0.3) (layers "F.Cu" "B.Cu") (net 1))
 (segment (start 197.25 112) (end 195 112) (width 0.4) (layer "B.Cu") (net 1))
 (segment (start 209.94 113.9) (end 209.94 112.4) (width 0.4) (layer "F.Cu") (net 12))
 (segment (start 207.34 116.5) (end 209.94 113.9) (width 0.4) (layer "F.Cu") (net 12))
 (segment (start 188 116.5) (end 207.34 116.5) (width 0.4) (layer "F.Cu") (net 12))
 (via (at 188 116.5) (size 0.6) (drill 0.3) (layers "F.Cu" "B.Cu") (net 12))
 (segment (start 181.5 110) (end 188 116.5) (width 0.4) (layer "B.Cu") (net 12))
 (segment (start 179 110) (end 181.5 110) (width 0.4) (layer "B.Cu") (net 12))
 (segment (start 206 110) (end 206.5 110) (width 0.4) (layer "F.Cu") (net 11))
 (segment (start 207.4 110.9) (end 207.4 112.4) (width 0.4) (layer "F.Cu") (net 11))
 (segment (start 206.5 110) (end 207.4 110.9) (width 0.4) (layer "F.Cu") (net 11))
 (via (at 206 110) (size 0.6) (drill 0.3) (layers "F.Cu" "B.Cu") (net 11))
 (segment (start 195 110) (end 206 110) (width 0.4) (layer "B.Cu") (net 11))
 (segment (start 204.86 109.36) (end 204.86 112.4) (width 0.4) (layer "F.Cu") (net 10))
 (segment (start 204 108.5) (end 204.86 109.36) (width 0.4) (layer "F.Cu") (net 10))
 (via (at 204 108.5) (size 0.6) (drill 0.3) (layers "F.Cu" "B.Cu") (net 10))
 (segment (start 204 108.5) (end 203.5 108) (width 0.4) (layer "B.Cu") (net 10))
 (segment (start 203.5 108) (end 195 108) (width 0.4) (layer "B.Cu") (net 10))
 (segment (start 202.32 107.32) (end 202.32 112.4) (width 0.4) (layer "F.Cu") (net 9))
 (segment (start 201 106) (end 202.32 107.32) (width 0.4) (layer "F.Cu") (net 9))
 (via (at 201 106) (size 0.6) (drill 0.3) (layers "F.Cu" "B.Cu") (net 9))
 (segment (start 195 106) (end 201 106) (width 0.4) (layer "B.Cu") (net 9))
 (segment (start 176 116) (end 172.42 112.42) (width 0.4) (layer "F.Cu") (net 14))
 (segment (start 215.02 112.4) (end 215.02 113.73) (width 0.4) (layer "F.Cu") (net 14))
 (segment (start 184.25 118) (end 182.25 116) (width 0.4) (layer "F.Cu") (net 14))
 (segment (start 208.75 118) (end 184.25 118) (width 0.4) (layer "F.Cu") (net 14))
 (segment (start 182.25 116) (end 176 116) (width 0.4) (layer "F.Cu") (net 14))
 (segment (start 172.42 112.42) (end 172.42 95.73) (width 0.4) (layer "F.Cu") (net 14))
 (segment (start 211.75 115) (end 208.75 118) (width 0.4) (layer "F.Cu") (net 14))
 (segment (start 213.75 115) (end 211.75 115) (width 0.4) (layer "F.Cu") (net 14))
 (segment (start 215.02 113.73) (end 213.75 115) (width 0.4) (layer "F.Cu") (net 14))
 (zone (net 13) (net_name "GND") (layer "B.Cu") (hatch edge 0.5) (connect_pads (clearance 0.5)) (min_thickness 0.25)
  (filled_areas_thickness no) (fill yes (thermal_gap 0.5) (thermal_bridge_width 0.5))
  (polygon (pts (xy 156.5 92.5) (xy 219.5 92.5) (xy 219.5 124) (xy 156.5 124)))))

